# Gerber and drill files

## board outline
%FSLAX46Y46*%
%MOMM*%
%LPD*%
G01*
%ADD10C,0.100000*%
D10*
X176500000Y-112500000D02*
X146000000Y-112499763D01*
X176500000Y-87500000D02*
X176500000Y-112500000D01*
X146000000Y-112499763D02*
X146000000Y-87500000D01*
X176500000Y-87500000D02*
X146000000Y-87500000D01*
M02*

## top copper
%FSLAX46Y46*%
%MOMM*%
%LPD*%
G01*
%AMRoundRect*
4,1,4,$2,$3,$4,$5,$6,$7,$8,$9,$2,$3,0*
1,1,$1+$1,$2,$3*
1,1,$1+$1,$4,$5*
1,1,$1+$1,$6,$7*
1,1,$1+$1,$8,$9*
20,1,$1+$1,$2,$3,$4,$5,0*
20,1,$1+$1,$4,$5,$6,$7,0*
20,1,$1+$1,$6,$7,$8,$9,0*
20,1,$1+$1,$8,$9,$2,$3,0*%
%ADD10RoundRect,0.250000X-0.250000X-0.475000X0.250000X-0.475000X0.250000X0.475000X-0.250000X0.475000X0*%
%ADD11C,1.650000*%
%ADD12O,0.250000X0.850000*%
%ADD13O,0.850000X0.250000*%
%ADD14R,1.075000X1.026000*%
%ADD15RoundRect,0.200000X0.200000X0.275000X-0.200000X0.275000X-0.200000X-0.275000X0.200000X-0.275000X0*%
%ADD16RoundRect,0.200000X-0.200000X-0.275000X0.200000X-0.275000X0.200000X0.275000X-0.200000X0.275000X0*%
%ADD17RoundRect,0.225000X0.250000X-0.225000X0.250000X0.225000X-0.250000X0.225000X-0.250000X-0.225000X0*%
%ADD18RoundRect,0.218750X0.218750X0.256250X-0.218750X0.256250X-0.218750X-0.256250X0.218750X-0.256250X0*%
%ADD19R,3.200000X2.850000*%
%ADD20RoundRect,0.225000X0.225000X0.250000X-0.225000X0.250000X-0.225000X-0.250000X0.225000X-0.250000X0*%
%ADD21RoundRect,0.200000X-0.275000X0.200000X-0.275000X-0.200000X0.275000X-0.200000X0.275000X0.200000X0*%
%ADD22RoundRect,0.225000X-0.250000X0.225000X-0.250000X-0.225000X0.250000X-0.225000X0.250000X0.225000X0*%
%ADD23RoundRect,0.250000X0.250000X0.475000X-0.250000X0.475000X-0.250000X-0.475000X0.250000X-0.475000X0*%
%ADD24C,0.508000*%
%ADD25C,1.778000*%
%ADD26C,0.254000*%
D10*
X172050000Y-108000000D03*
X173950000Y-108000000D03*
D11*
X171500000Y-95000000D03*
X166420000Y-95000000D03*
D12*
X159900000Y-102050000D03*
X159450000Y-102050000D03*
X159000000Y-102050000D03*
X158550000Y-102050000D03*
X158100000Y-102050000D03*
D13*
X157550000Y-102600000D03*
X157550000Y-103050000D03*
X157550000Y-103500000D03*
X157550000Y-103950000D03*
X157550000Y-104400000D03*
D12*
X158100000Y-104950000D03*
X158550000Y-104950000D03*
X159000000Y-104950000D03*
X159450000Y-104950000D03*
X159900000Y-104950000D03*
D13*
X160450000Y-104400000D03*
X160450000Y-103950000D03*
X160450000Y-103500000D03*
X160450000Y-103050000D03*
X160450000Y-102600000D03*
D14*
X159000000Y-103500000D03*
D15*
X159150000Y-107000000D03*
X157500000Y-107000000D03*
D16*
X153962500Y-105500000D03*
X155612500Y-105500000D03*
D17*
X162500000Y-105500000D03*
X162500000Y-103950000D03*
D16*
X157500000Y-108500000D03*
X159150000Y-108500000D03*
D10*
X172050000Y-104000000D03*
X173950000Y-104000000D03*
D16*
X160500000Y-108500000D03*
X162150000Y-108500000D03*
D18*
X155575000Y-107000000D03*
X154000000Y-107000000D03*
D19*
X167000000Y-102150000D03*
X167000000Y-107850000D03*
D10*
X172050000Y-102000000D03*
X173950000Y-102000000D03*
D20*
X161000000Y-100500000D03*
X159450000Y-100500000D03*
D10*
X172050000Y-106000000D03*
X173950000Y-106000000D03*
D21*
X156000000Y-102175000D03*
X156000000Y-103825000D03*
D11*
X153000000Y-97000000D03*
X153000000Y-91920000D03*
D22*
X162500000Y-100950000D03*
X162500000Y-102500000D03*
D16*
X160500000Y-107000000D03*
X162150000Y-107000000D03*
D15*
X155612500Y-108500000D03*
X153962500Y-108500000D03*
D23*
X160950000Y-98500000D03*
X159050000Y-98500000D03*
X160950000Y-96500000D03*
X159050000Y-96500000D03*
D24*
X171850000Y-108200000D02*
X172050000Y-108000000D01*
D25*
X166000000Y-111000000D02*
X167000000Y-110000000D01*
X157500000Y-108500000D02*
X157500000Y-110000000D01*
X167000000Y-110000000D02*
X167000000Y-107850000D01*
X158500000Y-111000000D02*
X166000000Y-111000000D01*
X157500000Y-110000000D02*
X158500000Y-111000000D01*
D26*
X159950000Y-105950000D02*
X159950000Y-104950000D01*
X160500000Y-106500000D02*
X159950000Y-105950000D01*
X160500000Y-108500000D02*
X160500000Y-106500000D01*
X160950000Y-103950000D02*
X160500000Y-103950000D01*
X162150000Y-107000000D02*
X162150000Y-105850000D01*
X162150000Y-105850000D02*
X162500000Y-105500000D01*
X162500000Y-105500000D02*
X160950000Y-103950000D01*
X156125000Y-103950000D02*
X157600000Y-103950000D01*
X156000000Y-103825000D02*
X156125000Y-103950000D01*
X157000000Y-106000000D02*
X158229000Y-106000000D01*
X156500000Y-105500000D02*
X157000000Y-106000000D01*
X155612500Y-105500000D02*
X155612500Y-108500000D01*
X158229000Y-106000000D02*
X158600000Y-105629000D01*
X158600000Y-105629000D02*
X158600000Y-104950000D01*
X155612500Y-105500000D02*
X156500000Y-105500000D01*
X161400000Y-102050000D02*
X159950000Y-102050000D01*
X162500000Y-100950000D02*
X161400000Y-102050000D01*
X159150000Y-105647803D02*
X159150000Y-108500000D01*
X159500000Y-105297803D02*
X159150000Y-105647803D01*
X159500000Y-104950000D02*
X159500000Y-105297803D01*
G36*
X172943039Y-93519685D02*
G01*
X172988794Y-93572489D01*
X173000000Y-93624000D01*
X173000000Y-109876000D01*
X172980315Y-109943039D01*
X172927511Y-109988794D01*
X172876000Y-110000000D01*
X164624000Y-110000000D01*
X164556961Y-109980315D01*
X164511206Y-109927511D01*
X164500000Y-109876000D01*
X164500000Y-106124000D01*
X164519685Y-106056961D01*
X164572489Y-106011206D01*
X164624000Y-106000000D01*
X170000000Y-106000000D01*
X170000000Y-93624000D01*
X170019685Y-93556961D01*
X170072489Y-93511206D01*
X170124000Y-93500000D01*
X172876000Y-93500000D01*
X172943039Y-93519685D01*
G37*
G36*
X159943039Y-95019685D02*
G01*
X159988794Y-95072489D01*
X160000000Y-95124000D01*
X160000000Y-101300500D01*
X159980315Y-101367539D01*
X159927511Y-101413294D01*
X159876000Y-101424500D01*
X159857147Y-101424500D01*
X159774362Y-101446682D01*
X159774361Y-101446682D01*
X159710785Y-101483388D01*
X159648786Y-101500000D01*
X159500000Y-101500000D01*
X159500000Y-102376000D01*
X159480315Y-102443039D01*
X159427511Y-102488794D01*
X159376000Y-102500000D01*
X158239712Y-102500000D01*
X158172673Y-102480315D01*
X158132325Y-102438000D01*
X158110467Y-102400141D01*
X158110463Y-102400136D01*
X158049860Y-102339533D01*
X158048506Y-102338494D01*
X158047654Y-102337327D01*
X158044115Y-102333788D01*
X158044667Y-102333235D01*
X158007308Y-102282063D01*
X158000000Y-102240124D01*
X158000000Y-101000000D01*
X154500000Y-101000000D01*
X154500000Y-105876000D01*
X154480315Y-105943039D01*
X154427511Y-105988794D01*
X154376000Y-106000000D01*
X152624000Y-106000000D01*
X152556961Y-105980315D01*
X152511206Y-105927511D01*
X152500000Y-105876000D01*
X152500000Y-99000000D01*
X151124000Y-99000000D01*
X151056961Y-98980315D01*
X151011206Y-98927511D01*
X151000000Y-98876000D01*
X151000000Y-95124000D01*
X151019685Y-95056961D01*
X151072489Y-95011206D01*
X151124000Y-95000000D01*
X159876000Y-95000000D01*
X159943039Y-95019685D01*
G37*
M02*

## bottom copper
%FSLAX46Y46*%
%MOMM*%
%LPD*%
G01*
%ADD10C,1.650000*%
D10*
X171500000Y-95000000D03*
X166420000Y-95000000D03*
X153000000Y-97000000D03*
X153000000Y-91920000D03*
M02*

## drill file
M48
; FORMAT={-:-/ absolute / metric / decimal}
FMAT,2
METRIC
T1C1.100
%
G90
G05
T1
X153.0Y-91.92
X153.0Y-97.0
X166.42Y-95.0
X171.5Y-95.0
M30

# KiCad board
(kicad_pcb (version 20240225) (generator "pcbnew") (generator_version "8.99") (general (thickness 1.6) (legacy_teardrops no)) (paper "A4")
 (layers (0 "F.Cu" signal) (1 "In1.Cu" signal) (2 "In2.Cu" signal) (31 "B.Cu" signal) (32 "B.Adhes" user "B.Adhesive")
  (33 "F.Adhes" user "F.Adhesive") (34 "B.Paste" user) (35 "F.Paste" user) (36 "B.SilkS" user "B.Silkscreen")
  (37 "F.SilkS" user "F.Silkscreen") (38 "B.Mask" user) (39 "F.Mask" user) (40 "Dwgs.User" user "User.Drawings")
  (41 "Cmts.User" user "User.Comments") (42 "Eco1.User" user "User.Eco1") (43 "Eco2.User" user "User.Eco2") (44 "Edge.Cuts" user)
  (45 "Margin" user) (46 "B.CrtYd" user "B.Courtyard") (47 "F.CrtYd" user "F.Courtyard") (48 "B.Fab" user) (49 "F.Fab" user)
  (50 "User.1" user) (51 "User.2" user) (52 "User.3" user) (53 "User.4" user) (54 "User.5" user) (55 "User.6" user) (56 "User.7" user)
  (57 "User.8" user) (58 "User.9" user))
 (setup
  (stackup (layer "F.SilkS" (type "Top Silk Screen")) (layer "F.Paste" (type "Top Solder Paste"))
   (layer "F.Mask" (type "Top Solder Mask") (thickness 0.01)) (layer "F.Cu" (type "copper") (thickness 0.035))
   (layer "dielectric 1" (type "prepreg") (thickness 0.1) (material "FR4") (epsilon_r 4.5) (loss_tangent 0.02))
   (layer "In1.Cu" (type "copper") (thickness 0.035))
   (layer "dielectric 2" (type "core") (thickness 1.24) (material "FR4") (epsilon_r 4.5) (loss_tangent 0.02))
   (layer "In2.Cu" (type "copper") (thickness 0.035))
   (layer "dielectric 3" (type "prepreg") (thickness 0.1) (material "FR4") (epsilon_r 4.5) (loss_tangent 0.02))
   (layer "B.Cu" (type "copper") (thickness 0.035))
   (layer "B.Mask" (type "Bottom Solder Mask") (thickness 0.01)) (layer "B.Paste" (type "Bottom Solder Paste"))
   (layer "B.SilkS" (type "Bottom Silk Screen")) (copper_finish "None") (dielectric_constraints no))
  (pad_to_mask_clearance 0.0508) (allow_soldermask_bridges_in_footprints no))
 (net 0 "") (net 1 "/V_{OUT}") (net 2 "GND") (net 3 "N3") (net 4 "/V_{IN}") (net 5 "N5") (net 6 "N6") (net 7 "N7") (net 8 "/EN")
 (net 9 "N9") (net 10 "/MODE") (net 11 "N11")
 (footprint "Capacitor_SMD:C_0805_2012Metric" (layer "F.Cu") (at 173 108)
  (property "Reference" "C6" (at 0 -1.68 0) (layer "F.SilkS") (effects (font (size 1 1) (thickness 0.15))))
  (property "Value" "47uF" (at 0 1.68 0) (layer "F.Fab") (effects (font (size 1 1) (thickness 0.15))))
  (pad "1" smd roundrect (at -0.95 0) (size 1 1.45) (layers "F.Cu" "F.Paste" "F.Mask") (roundrect_rratio 0.25) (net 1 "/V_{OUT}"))
  (pad "2" smd roundrect (at 0.95 0) (size 1 1.45) (layers "F.Cu" "F.Paste" "F.Mask") (roundrect_rratio 0.25) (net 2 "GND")))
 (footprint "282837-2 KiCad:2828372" (layer "F.Cu") (at 171.5 95 180)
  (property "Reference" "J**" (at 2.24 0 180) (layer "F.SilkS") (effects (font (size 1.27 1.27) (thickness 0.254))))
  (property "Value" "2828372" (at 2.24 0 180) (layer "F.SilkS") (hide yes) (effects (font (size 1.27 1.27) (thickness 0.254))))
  (pad "1" thru_hole circle (at 0 0 180) (size 1.65 1.65) (drill 1.1) (layers "*.Cu" "*.Mask") (remove_unused_layers no) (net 1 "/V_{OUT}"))
  (pad "2" thru_hole circle (at 5.08 0 180) (size 1.65 1.65) (drill 1.1) (layers "*.Cu" "*.Mask") (remove_unused_layers no) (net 2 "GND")))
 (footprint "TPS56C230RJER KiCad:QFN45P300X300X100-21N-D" (layer "F.Cu") (at 159 103.5 -90)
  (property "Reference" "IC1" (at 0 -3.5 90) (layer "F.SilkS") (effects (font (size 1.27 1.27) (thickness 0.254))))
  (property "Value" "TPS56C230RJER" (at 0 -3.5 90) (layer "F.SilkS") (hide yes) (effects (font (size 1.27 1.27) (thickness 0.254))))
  (pad "1" smd oval (at -1.45 -0.9) (size 0.25 0.85) (layers "F.Cu" "F.Paste" "F.Mask") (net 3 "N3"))
  (pad "2" smd oval (at -1.45 -0.45) (size 0.25 0.85) (layers "F.Cu" "F.Paste" "F.Mask") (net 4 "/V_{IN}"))
  (pad "3" smd oval (at -1.45 0) (size 0.25 0.85) (layers "F.Cu" "F.Paste" "F.Mask") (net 4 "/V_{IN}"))
  (pad "4" smd oval (at -1.45 0.45) (size 0.25 0.85) (layers "F.Cu" "F.Paste" "F.Mask") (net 4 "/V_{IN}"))
  (pad "5" smd oval (at -1.45 0.9) (size 0.25 0.85) (layers "F.Cu" "F.Paste" "F.Mask") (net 4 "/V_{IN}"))
  (pad "6" smd oval (at -0.9 1.45 270) (size 0.25 0.85) (layers "F.Cu" "F.Paste" "F.Mask") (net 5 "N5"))
  (pad "7" smd oval (at -0.45 1.45 270) (size 0.25 0.85) (layers "F.Cu" "F.Paste" "F.Mask") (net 2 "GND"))
  (pad "8" smd oval (at 0 1.45 270) (size 0.25 0.85) (layers "F.Cu" "F.Paste" "F.Mask") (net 2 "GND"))
  (pad "9" smd oval (at 0.45 1.45 270) (size 0.25 0.85) (layers "F.Cu" "F.Paste" "F.Mask") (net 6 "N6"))
  (pad "10" smd oval (at 0.9 1.45 270) (size 0.25 0.85) (layers "F.Cu" "F.Paste" "F.Mask") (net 2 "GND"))
  (pad "11" smd oval (at 1.45 0.9) (size 0.25 0.85) (layers "F.Cu" "F.Paste" "F.Mask") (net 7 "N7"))
  (pad "12" smd oval (at 1.45 0.45) (size 0.25 0.85) (layers "F.Cu" "F.Paste" "F.Mask") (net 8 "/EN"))
  (pad "13" smd oval (at 1.45 0) (size 0.25 0.85) (layers "F.Cu" "F.Paste" "F.Mask") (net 2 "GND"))
  (pad "14" smd oval (at 1.45 -0.45) (size 0.25 0.85) (layers "F.Cu" "F.Paste" "F.Mask") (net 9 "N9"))
  (pad "15" smd oval (at 1.45 -0.9) (size 0.25 0.85) (layers "F.Cu" "F.Paste" "F.Mask") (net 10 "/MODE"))
  (pad "16" smd oval (at 0.9 -1.45 270) (size 0.25 0.85) (layers "F.Cu" "F.Paste" "F.Mask") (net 2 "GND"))
  (pad "17" smd oval (at 0.45 -1.45 270) (size 0.25 0.85) (layers "F.Cu" "F.Paste" "F.Mask") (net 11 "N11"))
  (pad "18" smd oval (at 0 -1.45 270) (size 0.25 0.85) (layers "F.Cu" "F.Paste" "F.Mask") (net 2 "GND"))
  (pad "19" smd oval (at -0.45 -1.45 270) (size 0.25 0.85) (layers "F.Cu" "F.Paste" "F.Mask") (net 5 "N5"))
  (pad "20" smd oval (at -0.9 -1.45 270) (size 0.25 0.85) (layers "F.Cu" "F.Paste" "F.Mask") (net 5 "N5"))
  (pad "21" smd rect (at 0 0 270) (size 1.026 1.075) (layers "F.Cu" "F.Paste" "F.Mask") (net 2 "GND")))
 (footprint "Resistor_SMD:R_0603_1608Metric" (layer "F.Cu") (at 158.325 107 180)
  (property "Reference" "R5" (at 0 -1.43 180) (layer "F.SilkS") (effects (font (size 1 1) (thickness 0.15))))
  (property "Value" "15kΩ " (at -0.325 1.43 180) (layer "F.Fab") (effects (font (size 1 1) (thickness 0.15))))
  (pad "1" smd roundrect (at -0.825 0 180) (size 0.8 0.95) (layers "F.Cu" "F.Paste" "F.Mask") (roundrect_rratio 0.25) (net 9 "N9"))
  (pad "2" smd roundrect (at 0.825 0 180) (size 0.8 0.95) (layers "F.Cu" "F.Paste" "F.Mask") (roundrect_rratio 0.25) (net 2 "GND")))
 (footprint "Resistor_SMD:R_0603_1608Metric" (layer "F.Cu") (at 154.7875 105.5)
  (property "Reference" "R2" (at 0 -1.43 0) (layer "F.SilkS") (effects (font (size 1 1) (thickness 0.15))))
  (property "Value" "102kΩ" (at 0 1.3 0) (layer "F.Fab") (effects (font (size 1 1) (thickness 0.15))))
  (pad "1" smd roundrect (at -0.825 0) (size 0.8 0.95) (layers "F.Cu" "F.Paste" "F.Mask") (roundrect_rratio 0.25) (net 4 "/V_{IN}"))
  (pad "2" smd roundrect (at 0.825 0) (size 0.8 0.95) (layers "F.Cu" "F.Paste" "F.Mask") (roundrect_rratio 0.25) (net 8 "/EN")))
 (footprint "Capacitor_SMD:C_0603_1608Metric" (layer "F.Cu") (at 162.5 104.725 90)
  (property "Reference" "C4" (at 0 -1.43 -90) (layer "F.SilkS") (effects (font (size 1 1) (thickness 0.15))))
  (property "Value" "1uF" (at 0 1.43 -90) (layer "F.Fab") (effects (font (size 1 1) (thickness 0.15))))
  (pad "1" smd roundrect (at -0.775 0 90) (size 0.9 0.95) (layers "F.Cu" "F.Paste" "F.Mask") (roundrect_rratio 0.25) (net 11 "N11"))
  (pad "2" smd roundrect (at 0.775 0 90) (size 0.9 0.95) (layers "F.Cu" "F.Paste" "F.Mask") (roundrect_rratio 0.25) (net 2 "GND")))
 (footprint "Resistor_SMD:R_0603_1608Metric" (layer "F.Cu") (at 158.325 108.5)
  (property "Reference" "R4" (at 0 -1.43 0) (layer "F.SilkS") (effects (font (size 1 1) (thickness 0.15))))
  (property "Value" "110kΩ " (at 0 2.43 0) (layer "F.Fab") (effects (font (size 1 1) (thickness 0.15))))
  (pad "1" smd roundrect (at -0.825 0) (size 0.8 0.95) (layers "F.Cu" "F.Paste" "F.Mask") (roundrect_rratio 0.25) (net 1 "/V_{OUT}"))
  (pad "2" smd roundrect (at 0.825 0) (size 0.8 0.95) (layers "F.Cu" "F.Paste" "F.Mask") (roundrect_rratio 0.25) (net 9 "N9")))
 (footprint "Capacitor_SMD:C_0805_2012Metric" (layer "F.Cu") (at 173 104)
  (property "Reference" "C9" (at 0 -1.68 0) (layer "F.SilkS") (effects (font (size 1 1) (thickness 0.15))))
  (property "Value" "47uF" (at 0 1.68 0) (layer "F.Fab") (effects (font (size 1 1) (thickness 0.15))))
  (pad "1" smd roundrect (at -0.95 0) (size 1 1.45) (layers "F.Cu" "F.Paste" "F.Mask") (roundrect_rratio 0.25) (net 1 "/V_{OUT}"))
  (pad "2" smd roundrect (at 0.95 0) (size 1 1.45) (layers "F.Cu" "F.Paste" "F.Mask") (roundrect_rratio 0.25) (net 2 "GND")))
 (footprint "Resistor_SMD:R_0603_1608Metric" (layer "F.Cu") (at 161.325 108.5)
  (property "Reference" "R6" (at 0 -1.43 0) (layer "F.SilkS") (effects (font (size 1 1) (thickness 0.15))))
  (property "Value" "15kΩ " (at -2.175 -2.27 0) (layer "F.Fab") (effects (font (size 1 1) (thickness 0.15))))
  (pad "1" smd roundrect (at -0.825 0) (size 0.8 0.95) (layers "F.Cu" "F.Paste" "F.Mask") (roundrect_rratio 0.25) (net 10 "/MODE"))
  (pad "2" smd roundrect (at 0.825 0) (size 0.8 0.95) (layers "F.Cu" "F.Paste" "F.Mask") (roundrect_rratio 0.25) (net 2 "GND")))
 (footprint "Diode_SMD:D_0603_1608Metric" (layer "F.Cu") (at 154.7875 107 180)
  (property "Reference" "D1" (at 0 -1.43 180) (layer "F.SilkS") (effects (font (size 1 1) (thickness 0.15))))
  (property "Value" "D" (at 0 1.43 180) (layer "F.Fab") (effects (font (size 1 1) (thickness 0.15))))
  (pad "1" smd roundrect (at -0.7875 0 180) (size 0.875 0.95) (layers "F.Cu" "F.Paste" "F.Mask") (roundrect_rratio 0.25) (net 8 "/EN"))
  (pad "2" smd roundrect (at 0.7875 0 180) (size 0.875 0.95) (layers "F.Cu" "F.Paste" "F.Mask") (roundrect_rratio 0.25) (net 2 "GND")))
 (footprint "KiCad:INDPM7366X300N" (layer "F.Cu") (at 167 105 -90)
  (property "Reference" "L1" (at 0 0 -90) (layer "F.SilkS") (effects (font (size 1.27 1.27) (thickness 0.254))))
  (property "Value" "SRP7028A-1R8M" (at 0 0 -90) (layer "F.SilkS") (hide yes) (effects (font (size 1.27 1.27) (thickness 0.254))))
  (pad "1" smd rect (at -2.85 0 270) (size 2.85 3.2) (layers "F.Cu" "F.Paste" "F.Mask") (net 5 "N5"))
  (pad "2" smd rect (at 2.85 0 270) (size 2.85 3.2) (layers "F.Cu" "F.Paste" "F.Mask") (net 1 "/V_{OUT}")))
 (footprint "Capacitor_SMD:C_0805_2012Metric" (layer "F.Cu") (at 173 102)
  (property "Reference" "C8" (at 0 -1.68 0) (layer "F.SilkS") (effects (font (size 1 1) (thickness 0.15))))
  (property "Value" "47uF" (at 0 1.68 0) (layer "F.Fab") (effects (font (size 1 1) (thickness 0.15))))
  (pad "1" smd roundrect (at -0.95 0) (size 1 1.45) (layers "F.Cu" "F.Paste" "F.Mask") (roundrect_rratio 0.25) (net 1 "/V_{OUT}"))
  (pad "2" smd roundrect (at 0.95 0) (size 1 1.45) (layers "F.Cu" "F.Paste" "F.Mask") (roundrect_rratio 0.25) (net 2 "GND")))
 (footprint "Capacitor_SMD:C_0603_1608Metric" (layer "F.Cu") (at 160.225 100.5 180)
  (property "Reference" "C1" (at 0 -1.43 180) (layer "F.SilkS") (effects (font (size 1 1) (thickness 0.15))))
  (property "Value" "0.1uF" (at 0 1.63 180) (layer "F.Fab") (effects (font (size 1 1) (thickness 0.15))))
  (pad "1" smd roundrect (at -0.775 0 180) (size 0.9 0.95) (layers "F.Cu" "F.Paste" "F.Mask") (roundrect_rratio 0.25) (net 2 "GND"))
  (pad "2" smd roundrect (at 0.775 0 180) (size 0.9 0.95) (layers "F.Cu" "F.Paste" "F.Mask") (roundrect_rratio 0.25) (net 4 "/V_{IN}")))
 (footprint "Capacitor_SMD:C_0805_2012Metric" (layer "F.Cu") (at 173 106)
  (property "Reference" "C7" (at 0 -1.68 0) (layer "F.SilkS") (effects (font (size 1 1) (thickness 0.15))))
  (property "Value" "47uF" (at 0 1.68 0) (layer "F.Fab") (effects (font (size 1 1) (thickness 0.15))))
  (pad "1" smd roundrect (at -0.95 0) (size 1 1.45) (layers "F.Cu" "F.Paste" "F.Mask") (roundrect_rratio 0.25) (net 1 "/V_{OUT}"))
  (pad "2" smd roundrect (at 0.95 0) (size 1 1.45) (layers "F.Cu" "F.Paste" "F.Mask") (roundrect_rratio 0.25) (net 2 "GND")))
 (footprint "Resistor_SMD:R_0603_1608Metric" (layer "F.Cu") (at 156 103 -90)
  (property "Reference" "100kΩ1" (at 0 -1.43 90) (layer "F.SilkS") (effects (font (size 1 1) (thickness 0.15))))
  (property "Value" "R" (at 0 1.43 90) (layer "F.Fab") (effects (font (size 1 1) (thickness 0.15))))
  (pad "1" smd roundrect (at -0.825 0 270) (size 0.8 0.95) (layers "F.Cu" "F.Paste" "F.Mask") (roundrect_rratio 0.25) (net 11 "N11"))
  (pad "2" smd roundrect (at 0.825 0 270) (size 0.8 0.95) (layers "F.Cu" "F.Paste" "F.Mask") (roundrect_rratio 0.25) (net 6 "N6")))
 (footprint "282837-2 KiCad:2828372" (layer "F.Cu") (at 153 97 90)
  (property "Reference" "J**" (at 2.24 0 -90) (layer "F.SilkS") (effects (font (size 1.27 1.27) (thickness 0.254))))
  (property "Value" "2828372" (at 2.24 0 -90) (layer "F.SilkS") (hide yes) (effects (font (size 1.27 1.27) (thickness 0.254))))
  (pad "1" thru_hole circle (at 0 0 90) (size 1.65 1.65) (drill 1.1) (layers "*.Cu" "*.Mask") (remove_unused_layers no) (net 4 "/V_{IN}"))
  (pad "2" thru_hole circle (at 5.08 0 90) (size 1.65 1.65) (drill 1.1) (layers "*.Cu" "*.Mask") (remove_unused_layers no) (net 2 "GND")))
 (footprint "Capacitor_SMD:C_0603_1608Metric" (layer "F.Cu") (at 162.5 101.725 -90)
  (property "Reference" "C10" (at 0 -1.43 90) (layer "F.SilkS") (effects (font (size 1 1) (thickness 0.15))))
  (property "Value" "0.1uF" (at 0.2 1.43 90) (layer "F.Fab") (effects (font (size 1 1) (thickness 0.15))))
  (pad "1" smd roundrect (at -0.775 0 270) (size 0.9 0.95) (layers "F.Cu" "F.Paste" "F.Mask") (roundrect_rratio 0.25) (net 3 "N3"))
  (pad "2" smd roundrect (at 0.775 0 270) (size 0.9 0.95) (layers "F.Cu" "F.Paste" "F.Mask") (roundrect_rratio 0.25) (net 5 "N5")))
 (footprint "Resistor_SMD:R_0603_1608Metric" (layer "F.Cu") (at 161.325 107)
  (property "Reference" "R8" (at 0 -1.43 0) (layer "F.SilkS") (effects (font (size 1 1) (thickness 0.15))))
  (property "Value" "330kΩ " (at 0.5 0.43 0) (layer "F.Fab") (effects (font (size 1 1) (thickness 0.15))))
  (pad "1" smd roundrect (at -0.825 0) (size 0.8 0.95) (layers "F.Cu" "F.Paste" "F.Mask") (roundrect_rratio 0.25) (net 10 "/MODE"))
  (pad "2" smd roundrect (at 0.825 0) (size 0.8 0.95) (layers "F.Cu" "F.Paste" "F.Mask") (roundrect_rratio 0.25) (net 11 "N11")))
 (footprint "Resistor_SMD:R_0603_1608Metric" (layer "F.Cu") (at 154.7875 108.5 180)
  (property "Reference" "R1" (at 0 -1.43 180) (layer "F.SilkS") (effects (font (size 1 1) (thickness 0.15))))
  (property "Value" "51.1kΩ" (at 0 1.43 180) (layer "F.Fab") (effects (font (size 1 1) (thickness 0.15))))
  (pad "1" smd roundrect (at -0.825 0 180) (size 0.8 0.95) (layers "F.Cu" "F.Paste" "F.Mask") (roundrect_rratio 0.25) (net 8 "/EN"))
  (pad "2" smd roundrect (at 0.825 0 180) (size 0.8 0.95) (layers "F.Cu" "F.Paste" "F.Mask") (roundrect_rratio 0.25) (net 2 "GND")))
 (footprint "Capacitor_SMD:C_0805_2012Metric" (layer "F.Cu") (at 160 98.5 180)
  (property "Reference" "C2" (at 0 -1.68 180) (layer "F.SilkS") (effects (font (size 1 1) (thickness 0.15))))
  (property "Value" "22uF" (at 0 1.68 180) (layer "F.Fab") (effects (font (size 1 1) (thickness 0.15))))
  (pad "1" smd roundrect (at -0.95 0 180) (size 1 1.45) (layers "F.Cu" "F.Paste" "F.Mask") (roundrect_rratio 0.25) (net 2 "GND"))
  (pad "2" smd roundrect (at 0.95 0 180) (size 1 1.45) (layers "F.Cu" "F.Paste" "F.Mask") (roundrect_rratio 0.25) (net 4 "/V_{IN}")))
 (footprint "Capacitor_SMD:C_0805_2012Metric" (layer "F.Cu") (at 160 96.5 180)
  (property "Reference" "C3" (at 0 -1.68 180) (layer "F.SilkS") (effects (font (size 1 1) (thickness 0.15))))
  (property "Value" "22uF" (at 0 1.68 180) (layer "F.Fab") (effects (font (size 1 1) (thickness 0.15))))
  (pad "1" smd roundrect (at -0.95 0 180) (size 1 1.45) (layers "F.Cu" "F.Paste" "F.Mask") (roundrect_rratio 0.25) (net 2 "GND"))
  (pad "2" smd roundrect (at 0.95 0 180) (size 1 1.45) (layers "F.Cu" "F.Paste" "F.Mask") (roundrect_rratio 0.25) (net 4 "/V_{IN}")))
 (gr_line (start 176.5 112.5) (end 146 112.499763) (stroke (width 0.1) (type default)) (layer "Edge.Cuts"))
 (gr_line (start 176.5 87.5) (end 176.5 112.5) (stroke (width 0.1) (type default)) (layer "Edge.Cuts"))
 (gr_line (start 146 112.499763) (end 146 87.5) (stroke (width 0.1) (type default)) (layer "Edge.Cuts"))
 (gr_line (start 176.5 87.5) (end 146 87.5) (stroke (width 0.1) (type default)) (layer "Edge.Cuts"))
 (segment (start 171.85 108.2) (end 172.05 108) (width 0.508) (layer "F.Cu") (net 1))
 (segment (start 166 111) (end 167 110) (width 1.778) (layer "F.Cu") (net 1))
 (segment (start 157.5 108.5) (end 157.5 110) (width 1.778) (layer "F.Cu") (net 1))
 (segment (start 167 110) (end 167 107.85) (width 1.778) (layer "F.Cu") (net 1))
 (segment (start 158.5 111) (end 166 111) (width 1.778) (layer "F.Cu") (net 1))
 (segment (start 157.5 110) (end 158.5 111) (width 1.778) (layer "F.Cu") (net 1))
 (segment (start 159.95 105.95) (end 159.95 104.95) (width 0.254) (layer "F.Cu") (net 10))
 (segment (start 160.5 106.5) (end 159.95 105.95) (width 0.254) (layer "F.Cu") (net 10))
 (segment (start 160.5 108.5) (end 160.5 106.5) (width 0.254) (layer "F.Cu") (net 10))
 (segment (start 160.95 103.95) (end 160.5 103.95) (width 0.254) (layer "F.Cu") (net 11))
 (segment (start 162.15 107) (end 162.15 105.85) (width 0.254) (layer "F.Cu") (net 11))
 (segment (start 162.15 105.85) (end 162.5 105.5) (width 0.254) (layer "F.Cu") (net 11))
 (segment (start 162.5 105.5) (end 160.95 103.95) (width 0.254) (layer "F.Cu") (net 11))
 (segment (start 156.125 103.95) (end 157.6 103.95) (width 0.254) (layer "F.Cu") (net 6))
 (segment (start 156 103.825) (end 156.125 103.95) (width 0.254) (layer "F.Cu") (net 6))
 (segment (start 157 106) (end 158.229 106) (width 0.254) (layer "F.Cu") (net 8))
 (segment (start 156.5 105.5) (end 157 106) (width 0.254) (layer "F.Cu") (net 8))
 (segment (start 155.6125 105.5) (end 155.6125 108.5) (width 0.254) (layer "F.Cu") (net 8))
 (segment (start 158.229 106) (end 158.6 105.629) (width 0.254) (layer "F.Cu") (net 8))
 (segment (start 158.6 105.629) (end 158.6 104.95) (width 0.254) (layer "F.Cu") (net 8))
 (segment (start 155.6125 105.5) (end 156.5 105.5) (width 0.254) (layer "F.Cu") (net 8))
 (segment (start 161.4 102.05) (end 159.95 102.05) (width 0.254) (layer "F.Cu") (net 3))
 (segment (start 162.5 100.95) (end 161.4 102.05) (width 0.254) (layer "F.Cu") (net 3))
 (segment (start 159.15 105.647803) (end 159.15 108.5) (width 0.254) (layer "F.Cu") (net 9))
 (segment (start 159.5 105.297803) (end 159.15 105.647803) (width 0.254) (layer "F.Cu") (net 9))
 (segment (start 159.5 104.95) (end 159.5 105.297803) (width 0.254) (layer "F.Cu") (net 9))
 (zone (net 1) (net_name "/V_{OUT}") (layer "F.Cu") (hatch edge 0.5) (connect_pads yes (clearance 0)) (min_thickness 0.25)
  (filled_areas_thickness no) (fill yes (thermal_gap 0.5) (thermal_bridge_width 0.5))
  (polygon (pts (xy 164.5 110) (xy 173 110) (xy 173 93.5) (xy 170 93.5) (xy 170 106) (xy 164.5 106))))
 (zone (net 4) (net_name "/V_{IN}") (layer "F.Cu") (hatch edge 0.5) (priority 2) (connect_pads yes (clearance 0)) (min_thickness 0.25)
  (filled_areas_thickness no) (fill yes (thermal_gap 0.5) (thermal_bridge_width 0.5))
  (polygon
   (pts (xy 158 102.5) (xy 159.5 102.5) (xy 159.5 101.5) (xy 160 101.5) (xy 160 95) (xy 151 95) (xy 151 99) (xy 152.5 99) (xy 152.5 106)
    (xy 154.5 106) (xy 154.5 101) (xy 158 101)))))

